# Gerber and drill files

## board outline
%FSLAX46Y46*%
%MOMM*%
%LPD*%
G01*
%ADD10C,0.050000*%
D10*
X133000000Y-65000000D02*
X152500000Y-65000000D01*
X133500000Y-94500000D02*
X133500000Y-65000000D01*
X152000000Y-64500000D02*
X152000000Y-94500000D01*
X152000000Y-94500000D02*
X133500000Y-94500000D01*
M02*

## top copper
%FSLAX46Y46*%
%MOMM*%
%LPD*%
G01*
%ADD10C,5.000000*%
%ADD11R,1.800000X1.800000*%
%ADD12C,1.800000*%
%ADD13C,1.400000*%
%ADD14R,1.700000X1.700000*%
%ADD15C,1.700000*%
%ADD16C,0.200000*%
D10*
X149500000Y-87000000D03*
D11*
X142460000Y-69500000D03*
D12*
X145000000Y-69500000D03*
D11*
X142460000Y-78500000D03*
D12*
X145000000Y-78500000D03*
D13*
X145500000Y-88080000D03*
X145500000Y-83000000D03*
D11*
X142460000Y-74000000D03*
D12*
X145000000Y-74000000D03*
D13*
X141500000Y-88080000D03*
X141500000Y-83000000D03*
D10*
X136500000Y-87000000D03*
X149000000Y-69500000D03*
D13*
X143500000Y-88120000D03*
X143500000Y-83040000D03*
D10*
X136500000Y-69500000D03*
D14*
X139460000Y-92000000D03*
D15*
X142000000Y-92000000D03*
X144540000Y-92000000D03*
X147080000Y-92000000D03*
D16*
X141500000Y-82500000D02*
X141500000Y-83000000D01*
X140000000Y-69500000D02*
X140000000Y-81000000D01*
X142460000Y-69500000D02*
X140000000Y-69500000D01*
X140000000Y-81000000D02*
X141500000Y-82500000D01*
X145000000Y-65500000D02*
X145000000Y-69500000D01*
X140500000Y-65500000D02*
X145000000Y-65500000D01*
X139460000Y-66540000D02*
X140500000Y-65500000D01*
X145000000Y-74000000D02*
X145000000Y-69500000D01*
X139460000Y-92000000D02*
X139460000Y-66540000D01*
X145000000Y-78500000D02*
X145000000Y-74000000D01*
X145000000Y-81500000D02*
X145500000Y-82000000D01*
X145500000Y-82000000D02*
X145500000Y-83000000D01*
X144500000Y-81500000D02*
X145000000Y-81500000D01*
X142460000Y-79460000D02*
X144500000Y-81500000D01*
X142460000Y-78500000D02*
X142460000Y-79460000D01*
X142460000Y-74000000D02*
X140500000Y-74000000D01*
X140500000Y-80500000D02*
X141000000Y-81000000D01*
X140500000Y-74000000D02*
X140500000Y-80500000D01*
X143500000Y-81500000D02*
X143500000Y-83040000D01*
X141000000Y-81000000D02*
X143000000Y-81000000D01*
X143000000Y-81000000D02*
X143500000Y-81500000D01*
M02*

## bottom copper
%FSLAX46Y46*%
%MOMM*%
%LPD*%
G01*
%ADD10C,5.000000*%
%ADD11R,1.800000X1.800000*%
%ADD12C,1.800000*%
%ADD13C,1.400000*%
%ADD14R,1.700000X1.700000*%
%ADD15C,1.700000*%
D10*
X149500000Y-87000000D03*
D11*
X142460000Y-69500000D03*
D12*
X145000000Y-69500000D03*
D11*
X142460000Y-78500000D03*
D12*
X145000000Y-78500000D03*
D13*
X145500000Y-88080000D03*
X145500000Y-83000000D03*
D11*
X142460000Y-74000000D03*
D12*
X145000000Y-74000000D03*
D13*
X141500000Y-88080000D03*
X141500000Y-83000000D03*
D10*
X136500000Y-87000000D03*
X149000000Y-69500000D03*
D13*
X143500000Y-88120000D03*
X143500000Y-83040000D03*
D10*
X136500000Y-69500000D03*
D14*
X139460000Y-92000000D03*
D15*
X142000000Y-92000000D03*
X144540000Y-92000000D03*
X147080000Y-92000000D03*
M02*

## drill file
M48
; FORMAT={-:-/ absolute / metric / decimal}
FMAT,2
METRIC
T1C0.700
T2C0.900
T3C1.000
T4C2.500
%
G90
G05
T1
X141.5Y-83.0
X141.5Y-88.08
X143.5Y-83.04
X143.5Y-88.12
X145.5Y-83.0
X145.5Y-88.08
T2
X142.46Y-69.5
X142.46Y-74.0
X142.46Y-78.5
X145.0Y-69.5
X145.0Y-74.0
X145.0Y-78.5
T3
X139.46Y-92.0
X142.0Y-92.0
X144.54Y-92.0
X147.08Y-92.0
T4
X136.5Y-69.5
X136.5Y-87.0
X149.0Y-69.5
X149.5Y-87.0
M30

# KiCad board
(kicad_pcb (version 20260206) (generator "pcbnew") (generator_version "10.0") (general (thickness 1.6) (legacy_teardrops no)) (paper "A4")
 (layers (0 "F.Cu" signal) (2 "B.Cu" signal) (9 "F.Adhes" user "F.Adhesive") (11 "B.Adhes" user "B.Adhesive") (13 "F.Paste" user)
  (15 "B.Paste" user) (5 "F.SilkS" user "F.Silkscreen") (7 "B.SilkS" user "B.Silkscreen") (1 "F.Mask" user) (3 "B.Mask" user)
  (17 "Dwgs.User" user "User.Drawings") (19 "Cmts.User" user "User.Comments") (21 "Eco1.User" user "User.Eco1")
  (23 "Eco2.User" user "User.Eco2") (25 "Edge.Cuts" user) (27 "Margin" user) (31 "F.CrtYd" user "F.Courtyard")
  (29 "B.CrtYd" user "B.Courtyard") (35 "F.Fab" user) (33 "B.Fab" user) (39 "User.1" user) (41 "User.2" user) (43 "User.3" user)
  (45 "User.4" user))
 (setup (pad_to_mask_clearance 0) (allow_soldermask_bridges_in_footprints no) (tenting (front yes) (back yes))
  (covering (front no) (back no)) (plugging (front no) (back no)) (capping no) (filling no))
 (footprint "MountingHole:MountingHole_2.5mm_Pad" (layer "F.Cu") (at 149.5 87)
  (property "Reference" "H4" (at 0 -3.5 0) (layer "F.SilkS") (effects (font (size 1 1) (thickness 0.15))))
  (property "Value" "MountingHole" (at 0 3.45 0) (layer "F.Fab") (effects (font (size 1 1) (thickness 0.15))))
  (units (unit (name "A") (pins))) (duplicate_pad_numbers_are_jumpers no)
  (pad "1" thru_hole circle (at 0 0) (size 5 5) (drill 2.5) (layers "*.Cu" "*.Mask") (remove_unused_layers no) (zone_connect 2)))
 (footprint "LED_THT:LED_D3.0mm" (layer "F.Cu") (at 142.46 69.5)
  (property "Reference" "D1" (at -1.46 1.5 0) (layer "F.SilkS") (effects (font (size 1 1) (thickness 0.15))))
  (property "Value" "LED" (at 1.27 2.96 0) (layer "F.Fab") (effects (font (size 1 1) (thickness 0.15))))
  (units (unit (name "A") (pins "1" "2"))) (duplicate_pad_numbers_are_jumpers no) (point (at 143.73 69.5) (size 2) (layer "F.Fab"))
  (pad "1" thru_hole rect (at 0 0) (size 1.8 1.8) (drill 0.9) (layers "*.Cu" "*.Mask") (remove_unused_layers no) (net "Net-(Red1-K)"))
  (pad "2" thru_hole circle (at 2.54 0) (size 1.8 1.8) (drill 0.9) (layers "*.Cu" "*.Mask") (remove_unused_layers no) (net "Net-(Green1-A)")))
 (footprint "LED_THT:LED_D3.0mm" (layer "F.Cu") (at 142.46 78.5)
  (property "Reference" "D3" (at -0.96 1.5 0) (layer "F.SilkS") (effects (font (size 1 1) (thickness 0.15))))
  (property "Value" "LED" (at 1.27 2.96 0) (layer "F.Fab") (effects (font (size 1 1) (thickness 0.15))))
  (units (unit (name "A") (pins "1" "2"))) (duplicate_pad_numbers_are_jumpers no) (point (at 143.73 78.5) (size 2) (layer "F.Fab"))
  (pad "1" thru_hole rect (at 0 0) (size 1.8 1.8) (drill 0.9) (layers "*.Cu" "*.Mask") (remove_unused_layers no) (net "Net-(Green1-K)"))
  (pad "2" thru_hole circle (at 2.54 0) (size 1.8 1.8) (drill 0.9) (layers "*.Cu" "*.Mask") (remove_unused_layers no) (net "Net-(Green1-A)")))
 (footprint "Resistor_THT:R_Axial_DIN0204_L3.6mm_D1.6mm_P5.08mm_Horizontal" (layer "F.Cu") (at 145.5 88.08 90)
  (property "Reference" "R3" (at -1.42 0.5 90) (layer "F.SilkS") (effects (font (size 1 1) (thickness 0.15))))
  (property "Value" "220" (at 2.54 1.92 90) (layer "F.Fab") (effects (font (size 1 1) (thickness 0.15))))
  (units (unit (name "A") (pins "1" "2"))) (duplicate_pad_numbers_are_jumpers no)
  (pad "1" thru_hole circle (at 0 0 90) (size 1.4 1.4) (drill 0.7) (layers "*.Cu" "*.Mask") (remove_unused_layers no) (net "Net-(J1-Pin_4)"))
  (pad "2" thru_hole circle (at 5.08 0 90) (size 1.4 1.4) (drill 0.7) (layers "*.Cu" "*.Mask") (remove_unused_layers no)
   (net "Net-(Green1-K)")))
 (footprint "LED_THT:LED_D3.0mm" (layer "F.Cu") (at 142.46 74)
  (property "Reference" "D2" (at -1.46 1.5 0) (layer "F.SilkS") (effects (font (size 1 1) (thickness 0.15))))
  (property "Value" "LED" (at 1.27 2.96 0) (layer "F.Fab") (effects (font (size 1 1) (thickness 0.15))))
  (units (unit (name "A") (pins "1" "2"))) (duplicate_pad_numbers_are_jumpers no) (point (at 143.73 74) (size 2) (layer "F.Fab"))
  (pad "1" thru_hole rect (at 0 0) (size 1.8 1.8) (drill 0.9) (layers "*.Cu" "*.Mask") (remove_unused_layers no) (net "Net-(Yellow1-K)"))
  (pad "2" thru_hole circle (at 2.54 0) (size 1.8 1.8) (drill 0.9) (layers "*.Cu" "*.Mask") (remove_unused_layers no) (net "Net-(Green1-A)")))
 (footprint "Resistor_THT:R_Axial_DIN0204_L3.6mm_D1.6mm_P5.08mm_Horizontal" (layer "F.Cu") (at 141.5 88.08 90)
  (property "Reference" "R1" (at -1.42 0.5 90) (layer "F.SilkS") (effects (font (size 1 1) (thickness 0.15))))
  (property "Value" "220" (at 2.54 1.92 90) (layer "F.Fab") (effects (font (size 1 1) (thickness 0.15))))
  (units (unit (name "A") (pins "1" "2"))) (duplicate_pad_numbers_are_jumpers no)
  (pad "1" thru_hole circle (at 0 0 90) (size 1.4 1.4) (drill 0.7) (layers "*.Cu" "*.Mask") (remove_unused_layers no) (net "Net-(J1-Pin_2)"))
  (pad "2" thru_hole circle (at 5.08 0 90) (size 1.4 1.4) (drill 0.7) (layers "*.Cu" "*.Mask") (remove_unused_layers no)
   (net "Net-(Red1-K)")))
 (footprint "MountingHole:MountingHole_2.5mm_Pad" (layer "F.Cu") (at 136.5 87)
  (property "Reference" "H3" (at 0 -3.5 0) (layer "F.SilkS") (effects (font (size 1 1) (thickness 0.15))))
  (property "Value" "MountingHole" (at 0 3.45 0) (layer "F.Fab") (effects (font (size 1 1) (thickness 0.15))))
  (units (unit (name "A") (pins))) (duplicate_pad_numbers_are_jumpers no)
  (pad "1" thru_hole circle (at 0 0) (size 5 5) (drill 2.5) (layers "*.Cu" "*.Mask") (remove_unused_layers no) (zone_connect 2)))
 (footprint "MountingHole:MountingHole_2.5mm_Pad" (layer "F.Cu") (at 149 69.5)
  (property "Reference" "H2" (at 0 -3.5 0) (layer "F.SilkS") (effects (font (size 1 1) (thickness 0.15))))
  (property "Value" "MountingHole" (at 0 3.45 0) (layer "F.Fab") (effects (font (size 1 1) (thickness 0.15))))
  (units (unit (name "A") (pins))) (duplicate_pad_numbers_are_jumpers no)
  (pad "1" thru_hole circle (at 0 0) (size 5 5) (drill 2.5) (layers "*.Cu" "*.Mask") (remove_unused_layers no) (zone_connect 2)))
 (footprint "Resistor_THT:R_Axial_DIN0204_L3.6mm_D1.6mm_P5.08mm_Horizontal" (layer "F.Cu") (at 143.5 88.12 90)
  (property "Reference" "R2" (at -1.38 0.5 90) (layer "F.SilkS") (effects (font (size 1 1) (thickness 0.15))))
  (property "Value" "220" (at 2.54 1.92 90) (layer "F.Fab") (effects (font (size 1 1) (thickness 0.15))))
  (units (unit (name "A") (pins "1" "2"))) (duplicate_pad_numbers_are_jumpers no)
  (pad "1" thru_hole circle (at 0 0 90) (size 1.4 1.4) (drill 0.7) (layers "*.Cu" "*.Mask") (remove_unused_layers no) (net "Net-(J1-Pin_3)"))
  (pad "2" thru_hole circle (at 5.08 0 90) (size 1.4 1.4) (drill 0.7) (layers "*.Cu" "*.Mask") (remove_unused_layers no)
   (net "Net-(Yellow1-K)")))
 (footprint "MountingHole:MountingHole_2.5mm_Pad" (layer "F.Cu") (at 136.5 69.5)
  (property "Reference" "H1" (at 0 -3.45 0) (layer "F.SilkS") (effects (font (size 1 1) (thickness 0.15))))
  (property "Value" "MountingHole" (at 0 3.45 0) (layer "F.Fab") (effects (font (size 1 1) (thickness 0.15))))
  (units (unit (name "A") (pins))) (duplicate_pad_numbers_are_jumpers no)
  (pad "1" thru_hole circle (at 0 0) (size 5 5) (drill 2.5) (layers "*.Cu" "*.Mask") (remove_unused_layers no) (zone_connect 2)))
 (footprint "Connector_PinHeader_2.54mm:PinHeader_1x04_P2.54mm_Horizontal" (layer "B.Cu") (at 139.46 92 -90)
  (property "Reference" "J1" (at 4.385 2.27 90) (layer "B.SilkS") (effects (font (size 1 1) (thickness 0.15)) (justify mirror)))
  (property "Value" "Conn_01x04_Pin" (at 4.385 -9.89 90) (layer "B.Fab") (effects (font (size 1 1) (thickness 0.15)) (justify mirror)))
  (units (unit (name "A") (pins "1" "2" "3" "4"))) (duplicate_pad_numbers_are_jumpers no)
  (pad "1" thru_hole rect (at 0 0 270) (size 1.7 1.7) (drill 1) (layers "*.Cu" "*.Mask") (remove_unused_layers no) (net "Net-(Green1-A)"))
  (pad "2" thru_hole circle (at 0 -2.54 270) (size 1.7 1.7) (drill 1) (layers "*.Cu" "*.Mask") (remove_unused_layers no)
   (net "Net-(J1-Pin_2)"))
  (pad "3" thru_hole circle (at 0 -5.08 270) (size 1.7 1.7) (drill 1) (layers "*.Cu" "*.Mask") (remove_unused_layers no)
   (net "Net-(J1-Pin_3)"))
  (pad "4" thru_hole circle (at 0 -7.62 270) (size 1.7 1.7) (drill 1) (layers "*.Cu" "*.Mask") (remove_unused_layers no)
   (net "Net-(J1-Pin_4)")))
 (gr_line (start 133 65) (end 152.5 65) (stroke (width 0.05) (type default)) (layer "Edge.Cuts"))
 (gr_line (start 133.5 94.5) (end 133.5 65) (stroke (width 0.05) (type default)) (layer "Edge.Cuts"))
 (gr_line (start 152 64.5) (end 152 94.5) (stroke (width 0.05) (type default)) (layer "Edge.Cuts"))
 (gr_line (start 152 94.5) (end 133.5 94.5) (stroke (width 0.05) (type default)) (layer "Edge.Cuts"))
 (segment (start 141.5 82.5) (end 141.5 83) (width 0.2) (layer "F.Cu") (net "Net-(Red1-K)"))
 (segment (start 140 69.5) (end 140 81) (width 0.2) (layer "F.Cu") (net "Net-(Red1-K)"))
 (segment (start 142.46 69.5) (end 140 69.5) (width 0.2) (layer "F.Cu") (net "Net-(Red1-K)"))
 (segment (start 140 81) (end 141.5 82.5) (width 0.2) (layer "F.Cu") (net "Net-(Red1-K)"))
 (segment (start 145 65.5) (end 145 69.5) (width 0.2) (layer "F.Cu") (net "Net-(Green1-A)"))
 (segment (start 140.5 65.5) (end 145 65.5) (width 0.2) (layer "F.Cu") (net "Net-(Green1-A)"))
 (segment (start 139.46 66.54) (end 140.5 65.5) (width 0.2) (layer "F.Cu") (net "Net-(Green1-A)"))
 (segment (start 145 74) (end 145 69.5) (width 0.2) (layer "F.Cu") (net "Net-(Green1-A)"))
 (segment (start 139.46 92) (end 139.46 66.54) (width 0.2) (layer "F.Cu") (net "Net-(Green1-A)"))
 (segment (start 145 78.5) (end 145 74) (width 0.2) (layer "F.Cu") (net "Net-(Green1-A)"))
 (segment (start 145 81.5) (end 145.5 82) (width 0.2) (layer "F.Cu") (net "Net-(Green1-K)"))
 (segment (start 145.5 82) (end 145.5 83) (width 0.2) (layer "F.Cu") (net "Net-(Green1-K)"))
 (segment (start 144.5 81.5) (end 145 81.5) (width 0.2) (layer "F.Cu") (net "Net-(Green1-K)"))
 (segment (start 142.46 79.46) (end 144.5 81.5) (width 0.2) (layer "F.Cu") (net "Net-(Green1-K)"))
 (segment (start 142.46 78.5) (end 142.46 79.46) (width 0.2) (layer "F.Cu") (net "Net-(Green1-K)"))
 (segment (start 142.46 74) (end 140.5 74) (width 0.2) (layer "F.Cu") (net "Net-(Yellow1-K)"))
 (segment (start 140.5 80.5) (end 141 81) (width 0.2) (layer "F.Cu") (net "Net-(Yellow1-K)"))
 (segment (start 140.5 74) (end 140.5 80.5) (width 0.2) (layer "F.Cu") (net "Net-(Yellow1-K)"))
 (segment (start 143.5 81.5) (end 143.5 83.04) (width 0.2) (layer "F.Cu") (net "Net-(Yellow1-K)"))
 (segment (start 141 81) (end 143 81) (width 0.2) (layer "F.Cu") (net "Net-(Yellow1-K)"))
 (segment (start 143 81) (end 143.5 81.5) (width 0.2) (layer "F.Cu") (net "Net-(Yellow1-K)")))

